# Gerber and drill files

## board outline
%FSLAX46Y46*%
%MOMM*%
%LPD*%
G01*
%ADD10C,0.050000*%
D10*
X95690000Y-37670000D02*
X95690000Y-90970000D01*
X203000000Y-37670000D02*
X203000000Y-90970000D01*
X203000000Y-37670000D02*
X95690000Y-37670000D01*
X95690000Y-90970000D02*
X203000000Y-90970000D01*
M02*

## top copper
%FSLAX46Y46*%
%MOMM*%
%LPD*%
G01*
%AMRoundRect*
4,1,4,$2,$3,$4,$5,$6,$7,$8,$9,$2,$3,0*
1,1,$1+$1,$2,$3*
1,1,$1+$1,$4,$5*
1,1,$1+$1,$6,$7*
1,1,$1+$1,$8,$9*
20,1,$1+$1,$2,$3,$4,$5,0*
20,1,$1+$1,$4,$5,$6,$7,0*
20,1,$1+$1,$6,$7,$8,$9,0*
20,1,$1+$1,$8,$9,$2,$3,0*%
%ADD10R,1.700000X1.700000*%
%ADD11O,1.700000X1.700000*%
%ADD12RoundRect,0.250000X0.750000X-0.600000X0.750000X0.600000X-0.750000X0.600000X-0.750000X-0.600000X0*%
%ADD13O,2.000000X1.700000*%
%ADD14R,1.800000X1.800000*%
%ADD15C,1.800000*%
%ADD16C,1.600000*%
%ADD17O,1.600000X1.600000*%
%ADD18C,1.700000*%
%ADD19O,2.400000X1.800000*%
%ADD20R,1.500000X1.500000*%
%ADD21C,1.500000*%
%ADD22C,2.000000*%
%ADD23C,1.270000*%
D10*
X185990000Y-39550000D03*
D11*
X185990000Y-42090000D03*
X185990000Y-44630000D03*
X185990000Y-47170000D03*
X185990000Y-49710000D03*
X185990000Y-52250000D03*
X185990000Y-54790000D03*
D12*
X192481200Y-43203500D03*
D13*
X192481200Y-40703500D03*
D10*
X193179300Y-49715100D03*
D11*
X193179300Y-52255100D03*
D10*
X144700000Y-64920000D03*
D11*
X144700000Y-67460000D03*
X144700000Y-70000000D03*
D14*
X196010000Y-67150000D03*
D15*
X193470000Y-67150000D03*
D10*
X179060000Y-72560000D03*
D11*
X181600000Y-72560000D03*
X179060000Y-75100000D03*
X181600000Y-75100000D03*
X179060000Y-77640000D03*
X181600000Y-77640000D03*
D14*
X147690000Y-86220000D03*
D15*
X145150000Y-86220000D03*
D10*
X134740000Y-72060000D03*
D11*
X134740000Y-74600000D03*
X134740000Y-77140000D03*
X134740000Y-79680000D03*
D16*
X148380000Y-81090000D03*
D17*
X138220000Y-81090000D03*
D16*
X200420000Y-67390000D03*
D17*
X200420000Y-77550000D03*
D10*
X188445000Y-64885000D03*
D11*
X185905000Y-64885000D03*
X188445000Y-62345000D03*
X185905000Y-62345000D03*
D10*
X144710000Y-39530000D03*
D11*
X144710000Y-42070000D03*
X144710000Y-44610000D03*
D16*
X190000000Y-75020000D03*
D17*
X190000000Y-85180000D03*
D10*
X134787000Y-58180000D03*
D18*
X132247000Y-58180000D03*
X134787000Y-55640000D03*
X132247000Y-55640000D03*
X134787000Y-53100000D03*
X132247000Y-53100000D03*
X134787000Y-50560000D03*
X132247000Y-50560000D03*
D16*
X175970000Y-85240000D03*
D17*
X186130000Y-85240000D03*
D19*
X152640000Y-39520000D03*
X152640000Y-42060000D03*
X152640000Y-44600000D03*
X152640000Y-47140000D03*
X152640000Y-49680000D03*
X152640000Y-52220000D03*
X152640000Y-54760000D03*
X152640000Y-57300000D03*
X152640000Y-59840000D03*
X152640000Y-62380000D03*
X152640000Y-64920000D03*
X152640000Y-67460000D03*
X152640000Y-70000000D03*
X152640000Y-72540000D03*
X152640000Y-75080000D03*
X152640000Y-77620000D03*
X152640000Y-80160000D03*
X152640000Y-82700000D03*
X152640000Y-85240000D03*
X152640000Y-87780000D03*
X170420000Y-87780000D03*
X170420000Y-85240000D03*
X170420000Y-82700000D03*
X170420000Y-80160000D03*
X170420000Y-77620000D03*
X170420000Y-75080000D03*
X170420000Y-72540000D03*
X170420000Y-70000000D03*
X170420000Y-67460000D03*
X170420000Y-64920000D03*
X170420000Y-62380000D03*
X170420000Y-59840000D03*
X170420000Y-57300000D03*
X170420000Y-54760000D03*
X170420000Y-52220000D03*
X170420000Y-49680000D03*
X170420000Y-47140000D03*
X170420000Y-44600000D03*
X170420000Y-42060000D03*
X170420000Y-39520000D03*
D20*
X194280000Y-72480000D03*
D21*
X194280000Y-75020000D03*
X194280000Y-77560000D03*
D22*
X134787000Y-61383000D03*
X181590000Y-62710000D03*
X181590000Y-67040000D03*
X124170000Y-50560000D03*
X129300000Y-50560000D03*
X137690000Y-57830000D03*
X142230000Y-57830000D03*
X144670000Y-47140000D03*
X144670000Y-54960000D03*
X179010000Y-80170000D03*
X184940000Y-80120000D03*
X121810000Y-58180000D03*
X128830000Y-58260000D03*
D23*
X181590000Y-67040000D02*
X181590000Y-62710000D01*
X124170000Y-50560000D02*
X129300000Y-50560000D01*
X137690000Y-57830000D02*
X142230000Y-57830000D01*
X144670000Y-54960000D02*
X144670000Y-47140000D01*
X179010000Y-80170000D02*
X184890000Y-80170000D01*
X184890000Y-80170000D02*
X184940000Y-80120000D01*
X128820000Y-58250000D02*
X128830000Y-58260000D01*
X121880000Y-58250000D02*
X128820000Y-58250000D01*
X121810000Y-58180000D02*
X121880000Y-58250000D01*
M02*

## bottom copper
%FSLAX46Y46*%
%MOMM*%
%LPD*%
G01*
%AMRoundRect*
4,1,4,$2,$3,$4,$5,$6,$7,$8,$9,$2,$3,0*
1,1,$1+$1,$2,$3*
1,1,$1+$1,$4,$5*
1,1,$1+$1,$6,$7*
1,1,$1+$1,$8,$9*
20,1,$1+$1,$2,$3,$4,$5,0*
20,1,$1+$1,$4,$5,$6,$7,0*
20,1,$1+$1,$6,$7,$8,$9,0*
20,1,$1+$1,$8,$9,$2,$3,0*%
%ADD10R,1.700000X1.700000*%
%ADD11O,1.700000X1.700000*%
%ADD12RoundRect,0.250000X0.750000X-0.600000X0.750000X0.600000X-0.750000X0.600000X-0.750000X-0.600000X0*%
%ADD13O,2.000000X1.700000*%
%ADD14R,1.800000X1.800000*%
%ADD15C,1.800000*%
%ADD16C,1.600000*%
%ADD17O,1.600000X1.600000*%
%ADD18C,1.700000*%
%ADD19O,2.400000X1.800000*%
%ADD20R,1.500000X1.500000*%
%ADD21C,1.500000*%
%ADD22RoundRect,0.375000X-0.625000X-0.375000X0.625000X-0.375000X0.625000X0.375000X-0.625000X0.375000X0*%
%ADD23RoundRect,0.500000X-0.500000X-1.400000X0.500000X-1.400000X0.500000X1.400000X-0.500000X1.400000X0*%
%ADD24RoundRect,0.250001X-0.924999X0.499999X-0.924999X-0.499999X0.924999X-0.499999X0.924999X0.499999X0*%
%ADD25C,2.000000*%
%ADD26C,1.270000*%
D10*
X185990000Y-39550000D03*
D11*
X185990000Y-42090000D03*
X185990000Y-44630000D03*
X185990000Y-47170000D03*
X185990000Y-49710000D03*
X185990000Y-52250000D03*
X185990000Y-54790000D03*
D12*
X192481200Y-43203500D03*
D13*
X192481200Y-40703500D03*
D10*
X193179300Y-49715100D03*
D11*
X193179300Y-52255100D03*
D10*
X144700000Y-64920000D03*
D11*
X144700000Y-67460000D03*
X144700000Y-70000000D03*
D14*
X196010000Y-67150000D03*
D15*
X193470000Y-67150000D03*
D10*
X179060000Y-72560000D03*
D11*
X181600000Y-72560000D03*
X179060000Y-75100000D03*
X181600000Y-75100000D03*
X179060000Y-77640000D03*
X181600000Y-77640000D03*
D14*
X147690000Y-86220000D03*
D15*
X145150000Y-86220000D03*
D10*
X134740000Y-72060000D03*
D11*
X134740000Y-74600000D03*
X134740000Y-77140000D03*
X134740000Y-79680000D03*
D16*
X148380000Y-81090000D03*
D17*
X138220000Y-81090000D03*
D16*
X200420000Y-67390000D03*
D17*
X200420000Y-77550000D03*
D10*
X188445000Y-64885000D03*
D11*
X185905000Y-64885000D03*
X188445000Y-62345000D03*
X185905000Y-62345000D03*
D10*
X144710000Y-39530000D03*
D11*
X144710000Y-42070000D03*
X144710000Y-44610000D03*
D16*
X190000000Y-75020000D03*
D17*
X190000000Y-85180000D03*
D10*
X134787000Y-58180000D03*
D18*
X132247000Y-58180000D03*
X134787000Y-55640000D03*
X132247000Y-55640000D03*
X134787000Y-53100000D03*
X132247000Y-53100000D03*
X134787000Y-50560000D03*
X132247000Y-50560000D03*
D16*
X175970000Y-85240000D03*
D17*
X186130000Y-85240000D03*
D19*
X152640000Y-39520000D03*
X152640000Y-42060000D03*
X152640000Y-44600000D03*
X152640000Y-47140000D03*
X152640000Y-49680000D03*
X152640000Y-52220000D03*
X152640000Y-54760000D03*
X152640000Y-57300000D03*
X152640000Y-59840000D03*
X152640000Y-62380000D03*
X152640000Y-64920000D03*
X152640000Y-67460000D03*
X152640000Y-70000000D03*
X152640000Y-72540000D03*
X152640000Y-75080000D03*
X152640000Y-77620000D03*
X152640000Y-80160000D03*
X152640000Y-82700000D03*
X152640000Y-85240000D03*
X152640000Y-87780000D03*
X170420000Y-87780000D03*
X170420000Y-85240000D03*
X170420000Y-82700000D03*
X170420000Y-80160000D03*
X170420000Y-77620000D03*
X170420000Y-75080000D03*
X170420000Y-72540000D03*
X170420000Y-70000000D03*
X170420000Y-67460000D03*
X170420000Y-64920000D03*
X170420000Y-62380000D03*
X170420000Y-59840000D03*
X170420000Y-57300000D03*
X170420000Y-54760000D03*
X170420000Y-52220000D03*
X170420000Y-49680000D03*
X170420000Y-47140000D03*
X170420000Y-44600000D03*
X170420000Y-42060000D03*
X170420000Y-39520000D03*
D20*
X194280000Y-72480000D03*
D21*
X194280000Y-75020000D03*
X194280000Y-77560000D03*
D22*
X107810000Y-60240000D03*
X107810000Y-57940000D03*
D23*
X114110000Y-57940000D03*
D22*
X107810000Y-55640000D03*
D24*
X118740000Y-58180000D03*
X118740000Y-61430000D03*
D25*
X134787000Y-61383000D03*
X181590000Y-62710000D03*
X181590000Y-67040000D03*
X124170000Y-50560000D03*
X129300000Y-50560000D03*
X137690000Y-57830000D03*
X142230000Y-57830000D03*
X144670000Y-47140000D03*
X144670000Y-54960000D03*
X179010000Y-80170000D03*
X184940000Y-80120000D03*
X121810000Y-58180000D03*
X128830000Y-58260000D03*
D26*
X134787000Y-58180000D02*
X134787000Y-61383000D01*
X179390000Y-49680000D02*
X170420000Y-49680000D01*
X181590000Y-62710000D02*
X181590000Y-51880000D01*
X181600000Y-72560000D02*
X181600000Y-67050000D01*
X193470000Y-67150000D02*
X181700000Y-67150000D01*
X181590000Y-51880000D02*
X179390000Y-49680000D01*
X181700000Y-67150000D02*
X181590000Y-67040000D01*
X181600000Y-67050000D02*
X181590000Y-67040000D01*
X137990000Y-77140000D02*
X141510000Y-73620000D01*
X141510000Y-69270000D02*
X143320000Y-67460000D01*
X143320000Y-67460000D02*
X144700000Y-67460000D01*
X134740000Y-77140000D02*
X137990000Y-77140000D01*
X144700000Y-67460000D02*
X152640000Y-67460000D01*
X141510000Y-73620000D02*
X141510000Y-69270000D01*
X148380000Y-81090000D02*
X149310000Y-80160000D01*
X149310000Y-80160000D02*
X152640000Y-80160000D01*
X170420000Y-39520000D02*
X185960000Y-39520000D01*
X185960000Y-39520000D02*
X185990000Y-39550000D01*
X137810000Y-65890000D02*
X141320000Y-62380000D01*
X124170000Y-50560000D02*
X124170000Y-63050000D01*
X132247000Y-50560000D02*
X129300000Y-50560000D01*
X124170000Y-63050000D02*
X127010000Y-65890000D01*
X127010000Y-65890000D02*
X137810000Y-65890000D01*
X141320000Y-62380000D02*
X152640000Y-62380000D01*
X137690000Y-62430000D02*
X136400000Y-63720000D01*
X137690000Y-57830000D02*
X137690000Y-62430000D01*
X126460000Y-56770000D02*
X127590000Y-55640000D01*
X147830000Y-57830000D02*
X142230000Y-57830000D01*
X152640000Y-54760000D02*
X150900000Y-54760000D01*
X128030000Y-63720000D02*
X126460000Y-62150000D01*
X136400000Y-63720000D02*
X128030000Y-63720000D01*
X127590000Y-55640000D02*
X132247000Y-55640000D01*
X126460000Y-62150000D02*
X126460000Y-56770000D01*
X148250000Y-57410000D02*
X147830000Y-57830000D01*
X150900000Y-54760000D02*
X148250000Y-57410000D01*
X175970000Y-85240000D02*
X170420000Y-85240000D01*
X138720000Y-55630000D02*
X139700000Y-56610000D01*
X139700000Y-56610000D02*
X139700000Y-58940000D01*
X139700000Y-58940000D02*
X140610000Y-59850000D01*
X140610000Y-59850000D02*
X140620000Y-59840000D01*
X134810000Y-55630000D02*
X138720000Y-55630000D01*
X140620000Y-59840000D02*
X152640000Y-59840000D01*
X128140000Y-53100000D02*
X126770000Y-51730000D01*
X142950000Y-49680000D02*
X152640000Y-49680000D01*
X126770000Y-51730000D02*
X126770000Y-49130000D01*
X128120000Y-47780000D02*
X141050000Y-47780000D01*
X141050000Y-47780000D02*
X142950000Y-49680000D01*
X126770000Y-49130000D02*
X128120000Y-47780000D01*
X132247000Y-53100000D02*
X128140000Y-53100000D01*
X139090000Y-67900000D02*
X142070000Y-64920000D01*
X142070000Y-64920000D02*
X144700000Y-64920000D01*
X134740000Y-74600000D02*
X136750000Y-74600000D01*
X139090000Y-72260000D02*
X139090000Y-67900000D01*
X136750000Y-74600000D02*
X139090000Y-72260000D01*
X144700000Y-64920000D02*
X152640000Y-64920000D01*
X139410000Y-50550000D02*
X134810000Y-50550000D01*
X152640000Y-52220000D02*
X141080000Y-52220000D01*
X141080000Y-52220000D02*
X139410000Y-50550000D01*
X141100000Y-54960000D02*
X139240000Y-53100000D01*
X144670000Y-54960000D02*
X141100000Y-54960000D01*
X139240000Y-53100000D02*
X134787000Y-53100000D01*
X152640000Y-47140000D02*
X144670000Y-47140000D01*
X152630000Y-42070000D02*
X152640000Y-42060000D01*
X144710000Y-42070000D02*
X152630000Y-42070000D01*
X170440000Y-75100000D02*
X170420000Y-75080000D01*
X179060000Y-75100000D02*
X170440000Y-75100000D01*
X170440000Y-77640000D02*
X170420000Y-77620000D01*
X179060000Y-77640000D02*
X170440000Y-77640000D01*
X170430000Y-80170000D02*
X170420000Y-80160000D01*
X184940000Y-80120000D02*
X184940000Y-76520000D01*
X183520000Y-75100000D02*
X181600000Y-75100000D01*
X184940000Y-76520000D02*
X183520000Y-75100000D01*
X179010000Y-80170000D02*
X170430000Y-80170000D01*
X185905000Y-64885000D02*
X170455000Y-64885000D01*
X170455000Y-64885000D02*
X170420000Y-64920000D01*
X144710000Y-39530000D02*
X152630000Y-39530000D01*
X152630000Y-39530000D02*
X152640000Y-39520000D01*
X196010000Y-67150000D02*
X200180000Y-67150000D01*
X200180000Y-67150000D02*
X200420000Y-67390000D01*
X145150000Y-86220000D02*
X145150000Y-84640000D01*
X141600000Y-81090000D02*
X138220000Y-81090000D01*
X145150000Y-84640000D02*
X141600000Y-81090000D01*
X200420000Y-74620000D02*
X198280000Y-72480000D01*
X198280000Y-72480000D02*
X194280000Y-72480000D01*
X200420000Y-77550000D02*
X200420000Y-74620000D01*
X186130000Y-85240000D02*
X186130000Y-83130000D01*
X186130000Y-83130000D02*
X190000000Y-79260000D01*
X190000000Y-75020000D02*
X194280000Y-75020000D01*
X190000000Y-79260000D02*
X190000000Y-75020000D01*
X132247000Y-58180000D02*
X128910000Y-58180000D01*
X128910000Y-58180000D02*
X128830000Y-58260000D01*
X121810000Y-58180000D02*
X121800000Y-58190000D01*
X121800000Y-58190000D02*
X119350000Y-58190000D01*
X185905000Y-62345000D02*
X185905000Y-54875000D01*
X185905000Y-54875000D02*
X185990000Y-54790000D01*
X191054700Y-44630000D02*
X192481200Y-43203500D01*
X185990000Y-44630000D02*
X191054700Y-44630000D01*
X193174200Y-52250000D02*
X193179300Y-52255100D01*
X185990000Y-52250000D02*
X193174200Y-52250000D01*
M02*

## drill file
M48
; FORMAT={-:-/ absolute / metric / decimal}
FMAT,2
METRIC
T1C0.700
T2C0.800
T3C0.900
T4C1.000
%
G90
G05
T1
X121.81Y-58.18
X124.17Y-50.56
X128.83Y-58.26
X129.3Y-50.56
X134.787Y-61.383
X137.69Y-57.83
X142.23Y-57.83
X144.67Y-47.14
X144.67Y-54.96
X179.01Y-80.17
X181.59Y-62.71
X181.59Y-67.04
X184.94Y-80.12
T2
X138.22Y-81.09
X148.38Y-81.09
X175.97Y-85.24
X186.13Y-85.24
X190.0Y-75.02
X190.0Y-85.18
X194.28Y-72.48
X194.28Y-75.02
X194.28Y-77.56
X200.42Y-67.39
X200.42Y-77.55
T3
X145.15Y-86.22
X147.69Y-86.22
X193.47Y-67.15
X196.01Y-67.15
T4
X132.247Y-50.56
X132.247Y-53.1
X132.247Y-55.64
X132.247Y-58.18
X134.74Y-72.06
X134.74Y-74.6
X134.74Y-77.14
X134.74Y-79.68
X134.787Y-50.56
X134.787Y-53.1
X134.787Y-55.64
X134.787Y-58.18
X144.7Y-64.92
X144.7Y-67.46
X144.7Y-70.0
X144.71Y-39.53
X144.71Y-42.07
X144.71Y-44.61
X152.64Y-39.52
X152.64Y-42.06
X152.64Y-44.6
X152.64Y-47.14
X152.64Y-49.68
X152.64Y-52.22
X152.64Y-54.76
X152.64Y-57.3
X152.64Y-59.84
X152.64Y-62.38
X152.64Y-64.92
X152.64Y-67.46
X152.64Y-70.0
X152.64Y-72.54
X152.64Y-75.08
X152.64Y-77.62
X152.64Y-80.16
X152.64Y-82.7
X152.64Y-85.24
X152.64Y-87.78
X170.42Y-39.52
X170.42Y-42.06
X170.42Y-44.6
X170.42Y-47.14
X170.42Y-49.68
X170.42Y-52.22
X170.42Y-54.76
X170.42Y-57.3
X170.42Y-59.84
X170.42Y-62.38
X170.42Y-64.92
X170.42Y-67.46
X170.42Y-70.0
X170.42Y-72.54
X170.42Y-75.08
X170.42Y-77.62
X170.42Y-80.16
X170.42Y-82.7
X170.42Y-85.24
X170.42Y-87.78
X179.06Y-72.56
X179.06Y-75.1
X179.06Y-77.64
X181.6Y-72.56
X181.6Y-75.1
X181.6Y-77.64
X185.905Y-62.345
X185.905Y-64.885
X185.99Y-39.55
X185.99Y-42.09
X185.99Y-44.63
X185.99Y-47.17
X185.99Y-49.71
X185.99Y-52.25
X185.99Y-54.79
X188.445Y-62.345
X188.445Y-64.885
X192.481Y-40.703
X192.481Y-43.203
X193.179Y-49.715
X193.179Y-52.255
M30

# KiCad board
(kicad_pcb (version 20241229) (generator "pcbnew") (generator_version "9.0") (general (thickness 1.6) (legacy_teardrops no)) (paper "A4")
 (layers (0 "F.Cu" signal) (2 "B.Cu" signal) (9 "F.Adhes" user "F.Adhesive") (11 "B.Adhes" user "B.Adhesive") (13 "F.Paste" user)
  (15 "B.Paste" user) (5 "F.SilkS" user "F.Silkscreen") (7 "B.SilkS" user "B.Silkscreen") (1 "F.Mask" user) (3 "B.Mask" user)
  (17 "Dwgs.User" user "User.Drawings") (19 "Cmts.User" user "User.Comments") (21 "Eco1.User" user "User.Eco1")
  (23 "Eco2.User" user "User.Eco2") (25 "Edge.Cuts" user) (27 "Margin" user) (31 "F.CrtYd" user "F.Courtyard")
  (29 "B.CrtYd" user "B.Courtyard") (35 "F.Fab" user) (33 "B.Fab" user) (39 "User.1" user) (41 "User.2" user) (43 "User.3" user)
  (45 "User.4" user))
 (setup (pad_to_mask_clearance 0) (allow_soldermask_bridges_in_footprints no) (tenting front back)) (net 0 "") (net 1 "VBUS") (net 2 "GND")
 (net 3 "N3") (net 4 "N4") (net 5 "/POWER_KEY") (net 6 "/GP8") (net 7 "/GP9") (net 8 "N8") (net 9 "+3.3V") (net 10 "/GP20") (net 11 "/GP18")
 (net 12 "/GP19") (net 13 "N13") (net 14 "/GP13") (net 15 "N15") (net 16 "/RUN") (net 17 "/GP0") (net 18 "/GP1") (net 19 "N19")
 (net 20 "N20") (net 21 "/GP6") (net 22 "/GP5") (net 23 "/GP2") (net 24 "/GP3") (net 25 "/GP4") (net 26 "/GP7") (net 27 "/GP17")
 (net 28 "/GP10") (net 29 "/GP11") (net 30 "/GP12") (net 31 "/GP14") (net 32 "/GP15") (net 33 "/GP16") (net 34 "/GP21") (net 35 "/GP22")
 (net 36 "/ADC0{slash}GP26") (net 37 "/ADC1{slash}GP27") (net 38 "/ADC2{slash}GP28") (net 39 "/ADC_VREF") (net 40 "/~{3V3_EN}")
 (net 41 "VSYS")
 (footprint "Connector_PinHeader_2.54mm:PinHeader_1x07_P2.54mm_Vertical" (layer "F.Cu") (at 185.99 39.55)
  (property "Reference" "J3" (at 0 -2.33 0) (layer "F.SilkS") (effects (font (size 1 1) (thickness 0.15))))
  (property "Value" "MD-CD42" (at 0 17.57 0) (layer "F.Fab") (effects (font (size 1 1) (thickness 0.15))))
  (pad "1" thru_hole rect (at 0 0) (size 1.7 1.7) (drill 1) (layers "*.Cu" "*.Mask") (remove_unused_layers no) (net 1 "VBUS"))
  (pad "2" thru_hole oval (at 0 2.54) (size 1.7 1.7) (drill 1) (layers "*.Cu" "*.Mask") (remove_unused_layers no) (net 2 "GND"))
  (pad "3" thru_hole oval (at 0 5.08) (size 1.7 1.7) (drill 1) (layers "*.Cu" "*.Mask") (remove_unused_layers no) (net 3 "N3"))
  (pad "4" thru_hole oval (at 0 7.62) (size 1.7 1.7) (drill 1) (layers "*.Cu" "*.Mask") (remove_unused_layers no) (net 2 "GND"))
  (pad "5" thru_hole oval (at 0 10.16) (size 1.7 1.7) (drill 1) (layers "*.Cu" "*.Mask") (remove_unused_layers no) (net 2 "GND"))
  (pad "6" thru_hole oval (at 0 12.7) (size 1.7 1.7) (drill 1) (layers "*.Cu" "*.Mask") (remove_unused_layers no) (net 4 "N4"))
  (pad "7" thru_hole oval (at 0 15.24) (size 1.7 1.7) (drill 1) (layers "*.Cu" "*.Mask") (remove_unused_layers no) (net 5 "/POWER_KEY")))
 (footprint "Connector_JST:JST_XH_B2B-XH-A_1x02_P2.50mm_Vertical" (layer "F.Cu") (at 192.4812 43.2035 90)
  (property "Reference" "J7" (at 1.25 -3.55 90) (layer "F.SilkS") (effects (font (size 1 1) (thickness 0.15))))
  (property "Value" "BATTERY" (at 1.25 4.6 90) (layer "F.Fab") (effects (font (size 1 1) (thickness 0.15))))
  (pad "1" thru_hole roundrect (at 0 0 90) (size 1.7 2) (drill 1) (layers "*.Cu" "*.Mask") (remove_unused_layers no)
   (roundrect_rratio 0.147059) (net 3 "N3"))
  (pad "2" thru_hole oval (at 2.5 0 90) (size 1.7 2) (drill 1) (layers "*.Cu" "*.Mask") (remove_unused_layers no) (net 2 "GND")))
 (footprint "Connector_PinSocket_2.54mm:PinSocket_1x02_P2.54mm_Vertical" (layer "F.Cu") (at 193.1793 49.7151)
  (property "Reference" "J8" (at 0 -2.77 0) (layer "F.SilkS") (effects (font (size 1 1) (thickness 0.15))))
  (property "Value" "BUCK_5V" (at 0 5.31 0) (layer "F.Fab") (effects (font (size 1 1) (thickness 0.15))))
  (pad "1" thru_hole rect (at 0 0) (size 1.7 1.7) (drill 1) (layers "*.Cu" "*.Mask") (remove_unused_layers no) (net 2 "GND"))
  (pad "2" thru_hole oval (at 0 2.54) (size 1.7 1.7) (drill 1) (layers "*.Cu" "*.Mask") (remove_unused_layers no) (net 4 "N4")))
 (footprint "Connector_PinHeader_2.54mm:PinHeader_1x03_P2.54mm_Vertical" (layer "F.Cu") (at 144.7 64.92)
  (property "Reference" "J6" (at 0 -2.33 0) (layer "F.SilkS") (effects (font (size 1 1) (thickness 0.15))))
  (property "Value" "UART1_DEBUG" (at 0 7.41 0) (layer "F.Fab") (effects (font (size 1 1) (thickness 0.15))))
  (pad "1" thru_hole rect (at 0 0) (size 1.7 1.7) (drill 1) (layers "*.Cu" "*.Mask") (remove_unused_layers no) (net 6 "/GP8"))
  (pad "2" thru_hole oval (at 0 2.54) (size 1.7 1.7) (drill 1) (layers "*.Cu" "*.Mask") (remove_unused_layers no) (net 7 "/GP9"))
  (pad "3" thru_hole oval (at 0 5.08) (size 1.7 1.7) (drill 1) (layers "*.Cu" "*.Mask") (remove_unused_layers no) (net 2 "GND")))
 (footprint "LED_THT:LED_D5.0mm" (layer "F.Cu") (at 196.01 67.15 180)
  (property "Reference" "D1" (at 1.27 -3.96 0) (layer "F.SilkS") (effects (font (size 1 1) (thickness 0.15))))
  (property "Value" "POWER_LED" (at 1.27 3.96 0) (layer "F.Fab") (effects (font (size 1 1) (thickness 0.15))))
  (pad "1" thru_hole rect (at 0 0 180) (size 1.8 1.8) (drill 0.9) (layers "*.Cu" "*.Mask") (remove_unused_layers no) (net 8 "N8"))
  (pad "2" thru_hole circle (at 2.54 0 180) (size 1.8 1.8) (drill 0.9) (layers "*.Cu" "*.Mask") (remove_unused_layers no) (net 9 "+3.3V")))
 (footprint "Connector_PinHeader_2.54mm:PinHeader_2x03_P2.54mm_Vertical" (layer "F.Cu") (at 179.06 72.56)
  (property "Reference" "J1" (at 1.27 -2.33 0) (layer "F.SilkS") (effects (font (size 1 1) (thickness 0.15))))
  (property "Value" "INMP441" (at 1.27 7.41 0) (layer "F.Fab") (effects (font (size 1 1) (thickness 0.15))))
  (pad "1" thru_hole rect (at 0 0) (size 1.7 1.7) (drill 1) (layers "*.Cu" "*.Mask") (remove_unused_layers no) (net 2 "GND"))
  (pad "2" thru_hole oval (at 2.54 0) (size 1.7 1.7) (drill 1) (layers "*.Cu" "*.Mask") (remove_unused_layers no) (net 9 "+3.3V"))
  (pad "3" thru_hole oval (at 0 2.54) (size 1.7 1.7) (drill 1) (layers "*.Cu" "*.Mask") (remove_unused_layers no) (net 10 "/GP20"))
  (pad "4" thru_hole oval (at 2.54 2.54) (size 1.7 1.7) (drill 1) (layers "*.Cu" "*.Mask") (remove_unused_layers no) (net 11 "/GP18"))
  (pad "5" thru_hole oval (at 0 5.08) (size 1.7 1.7) (drill 1) (layers "*.Cu" "*.Mask") (remove_unused_layers no) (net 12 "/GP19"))
  (pad "6" thru_hole oval (at 2.54 5.08) (size 1.7 1.7) (drill 1) (layers "*.Cu" "*.Mask") (remove_unused_layers no) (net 2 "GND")))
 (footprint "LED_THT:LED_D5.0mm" (layer "F.Cu") (at 147.69 86.22 180)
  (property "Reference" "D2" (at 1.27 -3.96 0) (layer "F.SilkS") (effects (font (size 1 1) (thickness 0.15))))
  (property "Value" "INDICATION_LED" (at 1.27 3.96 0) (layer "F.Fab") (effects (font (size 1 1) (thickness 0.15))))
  (pad "1" thru_hole rect (at 0 0 180) (size 1.8 1.8) (drill 0.9) (layers "*.Cu" "*.Mask") (remove_unused_layers no) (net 2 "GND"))
  (pad "2" thru_hole circle (at 2.54 0 180) (size 1.8 1.8) (drill 0.9) (layers "*.Cu" "*.Mask") (remove_unused_layers no) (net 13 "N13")))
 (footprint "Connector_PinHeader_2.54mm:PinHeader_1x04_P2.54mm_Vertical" (layer "F.Cu") (at 134.74 72.06)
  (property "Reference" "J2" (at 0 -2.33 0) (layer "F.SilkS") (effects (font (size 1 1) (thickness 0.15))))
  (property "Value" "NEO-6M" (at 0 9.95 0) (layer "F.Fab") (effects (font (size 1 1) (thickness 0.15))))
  (pad "1" thru_hole rect (at 0 0) (size 1.7 1.7) (drill 1) (layers "*.Cu" "*.Mask") (remove_unused_layers no) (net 9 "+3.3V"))
  (pad "2" thru_hole oval (at 0 2.54) (size 1.7 1.7) (drill 1) (layers "*.Cu" "*.Mask") (remove_unused_layers no) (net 6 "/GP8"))
  (pad "3" thru_hole oval (at 0 5.08) (size 1.7 1.7) (drill 1) (layers "*.Cu" "*.Mask") (remove_unused_layers no) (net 7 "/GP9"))
  (pad "4" thru_hole oval (at 0 7.62) (size 1.7 1.7) (drill 1) (layers "*.Cu" "*.Mask") (remove_unused_layers no) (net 2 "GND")))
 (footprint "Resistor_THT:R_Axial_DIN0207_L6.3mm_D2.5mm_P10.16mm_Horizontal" (layer "F.Cu") (at 148.38 81.09 180)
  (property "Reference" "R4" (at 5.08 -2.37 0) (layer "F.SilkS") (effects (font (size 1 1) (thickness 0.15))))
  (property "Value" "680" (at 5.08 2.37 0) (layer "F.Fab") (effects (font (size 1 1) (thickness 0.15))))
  (pad "1" thru_hole circle (at 0 0 180) (size 1.6 1.6) (drill 0.8) (layers "*.Cu" "*.Mask") (remove_unused_layers no) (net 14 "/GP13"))
  (pad "2" thru_hole oval (at 10.16 0 180) (size 1.6 1.6) (drill 0.8) (layers "*.Cu" "*.Mask") (remove_unused_layers no) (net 13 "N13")))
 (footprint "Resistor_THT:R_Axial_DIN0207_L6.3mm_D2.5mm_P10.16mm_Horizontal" (layer "F.Cu") (at 200.42 67.39 -90)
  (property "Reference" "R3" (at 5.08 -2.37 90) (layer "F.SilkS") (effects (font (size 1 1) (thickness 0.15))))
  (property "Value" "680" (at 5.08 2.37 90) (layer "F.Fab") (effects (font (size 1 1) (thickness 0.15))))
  (pad "1" thru_hole circle (at 0 0 270) (size 1.6 1.6) (drill 0.8) (layers "*.Cu" "*.Mask") (remove_unused_layers no) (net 8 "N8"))
  (pad "2" thru_hole oval (at 10.16 0 270) (size 1.6 1.6) (drill 0.8) (layers "*.Cu" "*.Mask") (remove_unused_layers no) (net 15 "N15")))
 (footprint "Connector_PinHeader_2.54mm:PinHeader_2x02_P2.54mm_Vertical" (layer "F.Cu") (at 188.445 64.885 180)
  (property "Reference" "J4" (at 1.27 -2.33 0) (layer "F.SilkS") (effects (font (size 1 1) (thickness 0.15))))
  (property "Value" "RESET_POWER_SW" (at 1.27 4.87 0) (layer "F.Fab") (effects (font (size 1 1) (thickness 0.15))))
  (pad "1" thru_hole rect (at 0 0 180) (size 1.7 1.7) (drill 1) (layers "*.Cu" "*.Mask") (remove_unused_layers no) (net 2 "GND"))
  (pad "2" thru_hole oval (at 2.54 0 180) (size 1.7 1.7) (drill 1) (layers "*.Cu" "*.Mask") (remove_unused_layers no) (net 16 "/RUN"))
  (pad "3" thru_hole oval (at 0 2.54 180) (size 1.7 1.7) (drill 1) (layers "*.Cu" "*.Mask") (remove_unused_layers no) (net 2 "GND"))
  (pad "4" thru_hole oval (at 2.54 2.54 180) (size 1.7 1.7) (drill 1) (layers "*.Cu" "*.Mask") (remove_unused_layers no)
   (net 5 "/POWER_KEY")))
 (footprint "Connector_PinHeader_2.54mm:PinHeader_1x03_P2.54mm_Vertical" (layer "F.Cu") (at 144.71 39.53)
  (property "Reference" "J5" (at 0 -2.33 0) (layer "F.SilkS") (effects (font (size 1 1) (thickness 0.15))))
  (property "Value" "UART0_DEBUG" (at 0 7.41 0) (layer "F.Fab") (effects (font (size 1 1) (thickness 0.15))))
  (pad "1" thru_hole rect (at 0 0) (size 1.7 1.7) (drill 1) (layers "*.Cu" "*.Mask") (remove_unused_layers no) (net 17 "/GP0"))
  (pad "2" thru_hole oval (at 0 2.54) (size 1.7 1.7) (drill 1) (layers "*.Cu" "*.Mask") (remove_unused_layers no) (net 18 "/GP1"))
  (pad "3" thru_hole oval (at 0 5.08) (size 1.7 1.7) (drill 1) (layers "*.Cu" "*.Mask") (remove_unused_layers no) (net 2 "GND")))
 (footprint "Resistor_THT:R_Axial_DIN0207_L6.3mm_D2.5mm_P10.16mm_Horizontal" (layer "F.Cu") (at 190 75.02 -90)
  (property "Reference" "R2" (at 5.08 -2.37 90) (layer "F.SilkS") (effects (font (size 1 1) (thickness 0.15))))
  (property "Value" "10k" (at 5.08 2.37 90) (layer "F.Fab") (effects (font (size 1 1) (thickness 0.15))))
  (pad "1" thru_hole circle (at 0 0 270) (size 1.6 1.6) (drill 0.8) (layers "*.Cu" "*.Mask") (remove_unused_layers no) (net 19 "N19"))
  (pad "2" thru_hole oval (at 10.16 0 270) (size 1.6 1.6) (drill 0.8) (layers "*.Cu" "*.Mask") (remove_unused_layers no) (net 2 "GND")))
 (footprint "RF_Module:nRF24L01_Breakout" (layer "F.Cu") (at 136.287 54.39 180)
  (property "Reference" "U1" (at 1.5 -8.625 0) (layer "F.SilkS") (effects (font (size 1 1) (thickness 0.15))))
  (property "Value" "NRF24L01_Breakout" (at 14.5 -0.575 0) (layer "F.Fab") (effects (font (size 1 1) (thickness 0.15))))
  (pad "1" thru_hole rect (at 1.5 -3.79 180) (size 1.7 1.7) (drill 1) (layers "*.Cu" "*.Mask") (remove_unused_layers no) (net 2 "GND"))
  (pad "2" thru_hole circle (at 4.04 -3.79 180) (size 1.7 1.7) (drill 1) (layers "*.Cu" "*.Mask") (remove_unused_layers no) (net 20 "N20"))
  (pad "3" thru_hole circle (at 1.5 -1.25 180) (size 1.7 1.7) (drill 1) (layers "*.Cu" "*.Mask") (remove_unused_layers no) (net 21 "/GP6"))
  (pad "4" thru_hole circle (at 4.04 -1.25 180) (size 1.7 1.7) (drill 1) (layers "*.Cu" "*.Mask") (remove_unused_layers no) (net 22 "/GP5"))
  (pad "5" thru_hole circle (at 1.5 1.29 180) (size 1.7 1.7) (drill 1) (layers "*.Cu" "*.Mask") (remove_unused_layers no) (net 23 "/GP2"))
  (pad "6" thru_hole circle (at 4.04 1.29 180) (size 1.7 1.7) (drill 1) (layers "*.Cu" "*.Mask") (remove_unused_layers no) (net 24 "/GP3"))
  (pad "7" thru_hole circle (at 1.5 3.83 180) (size 1.7 1.7) (drill 1) (layers "*.Cu" "*.Mask") (remove_unused_layers no) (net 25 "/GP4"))
  (pad "8" thru_hole circle (at 4.04 3.83 180) (size 1.7 1.7) (drill 1) (layers "*.Cu" "*.Mask") (remove_unused_layers no) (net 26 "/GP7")))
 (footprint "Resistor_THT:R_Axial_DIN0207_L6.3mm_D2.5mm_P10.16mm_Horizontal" (layer "F.Cu") (at 175.97 85.24)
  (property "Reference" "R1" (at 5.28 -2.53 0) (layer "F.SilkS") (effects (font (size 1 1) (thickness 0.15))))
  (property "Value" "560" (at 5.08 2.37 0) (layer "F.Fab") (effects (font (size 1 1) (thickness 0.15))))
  (pad "1" thru_hole circle (at 0 0) (size 1.6 1.6) (drill 0.8) (layers "*.Cu" "*.Mask") (remove_unused_layers no) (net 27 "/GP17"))
  (pad "2" thru_hole oval (at 10.16 0) (size 1.6 1.6) (drill 0.8) (layers "*.Cu" "*.Mask") (remove_unused_layers no) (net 19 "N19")))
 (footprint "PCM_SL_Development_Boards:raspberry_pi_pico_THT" (layer "F.Cu") (at 152.64 39.52)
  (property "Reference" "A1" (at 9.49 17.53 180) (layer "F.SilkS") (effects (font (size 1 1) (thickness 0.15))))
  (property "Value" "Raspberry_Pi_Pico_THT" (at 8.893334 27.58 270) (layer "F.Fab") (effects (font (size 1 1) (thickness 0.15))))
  (pad "1" thru_hole oval (at 0 0 270) (size 1.8 2.4) (drill 1) (layers "*.Cu" "*.Mask") (remove_unused_layers no) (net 17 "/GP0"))
  (pad "2" thru_hole oval (at 0 2.54 270) (size 1.8 2.4) (drill 1) (layers "*.Cu" "*.Mask") (remove_unused_layers no) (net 18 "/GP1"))
  (pad "3" thru_hole oval (at 0 5.08 270) (size 1.8 2.4) (drill 1) (layers "*.Cu" "*.Mask") (remove_unused_layers no) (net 2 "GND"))
  (pad "4" thru_hole oval (at 0 7.62 270) (size 1.8 2.4) (drill 1) (layers "*.Cu" "*.Mask") (remove_unused_layers no) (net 23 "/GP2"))
  (pad "5" thru_hole oval (at 0 10.16 270) (size 1.8 2.4) (drill 1) (layers "*.Cu" "*.Mask") (remove_unused_layers no) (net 24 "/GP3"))
  (pad "6" thru_hole oval (at 0 12.7 270) (size 1.8 2.4) (drill 1) (layers "*.Cu" "*.Mask") (remove_unused_layers no) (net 25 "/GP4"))
  (pad "7" thru_hole oval (at 0 15.24 270) (size 1.8 2.4) (drill 1) (layers "*.Cu" "*.Mask") (remove_unused_layers no) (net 22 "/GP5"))
  (pad "8" thru_hole oval (at 0 17.78 270) (size 1.8 2.4) (drill 1) (layers "*.Cu" "*.Mask") (remove_unused_layers no) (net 2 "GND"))
  (pad "9" thru_hole oval (at 0 20.32 270) (size 1.8 2.4) (drill 1) (layers "*.Cu" "*.Mask") (remove_unused_layers no) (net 21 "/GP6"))
  (pad "10" thru_hole oval (at 0 22.86 270) (size 1.8 2.4) (drill 1) (layers "*.Cu" "*.Mask") (remove_unused_layers no) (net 26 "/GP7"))
  (pad "11" thru_hole oval (at 0 25.4 270) (size 1.8 2.4) (drill 1) (layers "*.Cu" "*.Mask") (remove_unused_layers no) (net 6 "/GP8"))
  (pad "12" thru_hole oval (at 0 27.94 270) (size 1.8 2.4) (drill 1) (layers "*.Cu" "*.Mask") (remove_unused_layers no) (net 7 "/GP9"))
  (pad "13" thru_hole oval (at 0 30.48 270) (size 1.8 2.4) (drill 1) (layers "*.Cu" "*.Mask") (remove_unused_layers no) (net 2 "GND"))
  (pad "14" thru_hole oval (at 0 33.02 270) (size 1.8 2.4) (drill 1) (layers "*.Cu" "*.Mask") (remove_unused_layers no) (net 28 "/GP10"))
  (pad "15" thru_hole oval (at 0 35.56 270) (size 1.8 2.4) (drill 1) (layers "*.Cu" "*.Mask") (remove_unused_layers no) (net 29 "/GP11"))
  (pad "16" thru_hole oval (at 0 38.1 270) (size 1.8 2.4) (drill 1) (layers "*.Cu" "*.Mask") (remove_unused_layers no) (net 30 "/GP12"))
  (pad "17" thru_hole oval (at 0 40.64 270) (size 1.8 2.4) (drill 1) (layers "*.Cu" "*.Mask") (remove_unused_layers no) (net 14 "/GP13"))
  (pad "18" thru_hole oval (at 0 43.18 270) (size 1.8 2.4) (drill 1) (layers "*.Cu" "*.Mask") (remove_unused_layers no) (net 2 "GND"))
  (pad "19" thru_hole oval (at 0 45.72 270) (size 1.8 2.4) (drill 1) (layers "*.Cu" "*.Mask") (remove_unused_layers no) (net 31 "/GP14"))
  (pad "20" thru_hole oval (at 0 48.26 270) (size 1.8 2.4) (drill 1) (layers "*.Cu" "*.Mask") (remove_unused_layers no) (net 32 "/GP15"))
  (pad "21" thru_hole oval (at 17.78 48.26 270) (size 1.8 2.4) (drill 1) (layers "*.Cu" "*.Mask") (remove_unused_layers no) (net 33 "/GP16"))
  (pad "22" thru_hole oval (at 17.78 45.72 270) (size 1.8 2.4) (drill 1) (layers "*.Cu" "*.Mask") (remove_unused_layers no) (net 27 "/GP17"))
  (pad "23" thru_hole oval (at 17.78 43.18 270) (size 1.8 2.4) (drill 1) (layers "*.Cu" "*.Mask") (remove_unused_layers no) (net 2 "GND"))
  (pad "24" thru_hole oval (at 17.78 40.64 270) (size 1.8 2.4) (drill 1) (layers "*.Cu" "*.Mask") (remove_unused_layers no) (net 11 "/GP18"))
  (pad "25" thru_hole oval (at 17.78 38.1 270) (size 1.8 2.4) (drill 1) (layers "*.Cu" "*.Mask") (remove_unused_layers no) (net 12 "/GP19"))
  (pad "26" thru_hole oval (at 17.78 35.56 270) (size 1.8 2.4) (drill 1) (layers "*.Cu" "*.Mask") (remove_unused_layers no) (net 10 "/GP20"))
  (pad "27" thru_hole oval (at 17.78 33.02 270) (size 1.8 2.4) (drill 1) (layers "*.Cu" "*.Mask") (remove_unused_layers no) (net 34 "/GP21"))
  (pad "28" thru_hole oval (at 17.78 30.48 270) (size 1.8 2.4) (drill 1) (layers "*.Cu" "*.Mask") (remove_unused_layers no) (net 2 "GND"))
  (pad "29" thru_hole oval (at 17.78 27.94 270) (size 1.8 2.4) (drill 1) (layers "*.Cu" "*.Mask") (remove_unused_layers no) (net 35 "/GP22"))
  (pad "30" thru_hole oval (at 17.78 25.4 270) (size 1.8 2.4) (drill 1) (layers "*.Cu" "*.Mask") (remove_unused_layers no) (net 16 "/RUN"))
  (pad "31" thru_hole oval (at 17.78 22.86 270) (size 1.8 2.4) (drill 1) (layers "*.Cu" "*.Mask") (remove_unused_layers no)
   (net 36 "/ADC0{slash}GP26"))
  (pad "32" thru_hole oval (at 17.78 20.32 270) (size 1.8 2.4) (drill 1) (layers "*.Cu" "*.Mask") (remove_unused_layers no)
   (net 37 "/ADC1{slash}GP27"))
  (pad "33" thru_hole oval (at 17.78 17.78 270) (size 1.8 2.4) (drill 1) (layers "*.Cu" "*.Mask") (remove_unused_layers no) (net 2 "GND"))
  (pad "34" thru_hole oval (at 17.78 15.24 270) (size 1.8 2.4) (drill 1) (layers "*.Cu" "*.Mask") (remove_unused_layers no)
   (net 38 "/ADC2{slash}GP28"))
  (pad "35" thru_hole oval (at 17.78 12.7 270) (size 1.8 2.4) (drill 1) (layers "*.Cu" "*.Mask") (remove_unused_layers no)
   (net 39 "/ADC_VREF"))
  (pad "36" thru_hole oval (at 17.78 10.16 270) (size 1.8 2.4) (drill 1) (layers "*.Cu" "*.Mask") (remove_unused_layers no) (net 9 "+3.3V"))
  (pad "37" thru_hole oval (at 17.78 7.62 270) (size 1.8 2.4) (drill 1) (layers "*.Cu" "*.Mask") (remove_unused_layers no)
   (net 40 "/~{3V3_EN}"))
  (pad "38" thru_hole oval (at 17.78 5.08 270) (size 1.8 2.4) (drill 1) (layers "*.Cu" "*.Mask") (remove_unused_layers no) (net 2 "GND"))
  (pad "39" thru_hole oval (at 17.78 2.54 270) (size 1.8 2.4) (drill 1) (layers "*.Cu" "*.Mask") (remove_unused_layers no) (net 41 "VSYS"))
  (pad "40" thru_hole oval (at 17.78 0 270) (size 1.8 2.4) (drill 1) (layers "*.Cu" "*.Mask") (remove_unused_layers no) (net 1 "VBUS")))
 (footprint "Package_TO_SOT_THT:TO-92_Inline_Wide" (layer "F.Cu") (at 194.28 72.48 -90)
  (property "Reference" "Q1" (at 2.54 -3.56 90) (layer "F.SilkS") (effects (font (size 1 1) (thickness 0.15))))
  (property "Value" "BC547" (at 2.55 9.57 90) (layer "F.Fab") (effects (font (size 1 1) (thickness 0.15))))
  (pad "1" thru_hole rect (at 0 0 270) (size 1.5 1.5) (drill 0.8) (layers "*.Cu" "*.Mask") (remove_unused_layers no) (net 15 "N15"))
  (pad "2" thru_hole circle (at 2.54 0 270) (size 1.5 1.5) (drill 0.8) (layers "*.Cu" "*.Mask") (remove_unused_layers no) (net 19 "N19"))
  (pad "3" thru_hole circle (at 5.08 0 270) (size 1.5 1.5) (drill 0.8) (layers "*.Cu" "*.Mask") (remove_unused_layers no) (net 2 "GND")))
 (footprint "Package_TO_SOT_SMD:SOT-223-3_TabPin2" (layer "B.Cu") (at 110.96 57.94)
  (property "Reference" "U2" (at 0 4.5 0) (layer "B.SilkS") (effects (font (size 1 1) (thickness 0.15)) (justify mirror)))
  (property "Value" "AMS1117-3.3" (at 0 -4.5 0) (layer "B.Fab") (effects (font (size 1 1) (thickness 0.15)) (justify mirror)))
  (pad "1" smd roundrect (at -3.15 2.3) (size 2 1.5) (layers "B.Cu" "B.Mask" "B.Paste") (roundrect_rratio 0.25) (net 2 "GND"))
  (pad "2" smd roundrect (at -3.15 0) (size 2 1.5) (layers "B.Cu" "B.Mask" "B.Paste") (roundrect_rratio 0.25) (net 20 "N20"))
  (pad "2" smd roundrect (at 3.15 0) (size 2 3.8) (layers "B.Cu" "B.Mask" "B.Paste") (roundrect_rratio 0.25) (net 20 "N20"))
  (pad "3" smd roundrect (at -3.15 -2.3) (size 2 1.5) (layers "B.Cu" "B.Mask" "B.Paste") (roundrect_rratio 0.25) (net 1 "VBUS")))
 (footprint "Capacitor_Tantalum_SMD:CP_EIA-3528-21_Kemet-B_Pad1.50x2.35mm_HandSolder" (layer "B.Cu") (at 118.74 59.805 -90)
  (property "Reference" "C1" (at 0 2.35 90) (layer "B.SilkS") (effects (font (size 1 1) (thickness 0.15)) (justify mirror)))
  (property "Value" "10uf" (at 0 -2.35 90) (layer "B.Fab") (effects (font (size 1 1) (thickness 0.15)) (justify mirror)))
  (pad "1" smd roundrect (at -1.625 0 270) (size 1.5 2.35) (layers "B.Cu" "B.Mask" "B.Paste") (roundrect_rratio 0.166667) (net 20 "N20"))
  (pad "2" smd roundrect (at 1.625 0 270) (size 1.5 2.35) (layers "B.Cu" "B.Mask" "B.Paste") (roundrect_rratio 0.166667) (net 2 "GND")))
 (gr_line (start 95.69 37.67) (end 95.69 90.97) (stroke (width 0.05) (type default)) (layer "Edge.Cuts"))
 (gr_line (start 203 37.67) (end 203 90.97) (stroke (width 0.05) (type default)) (layer "Edge.Cuts"))
 (gr_line (start 203 37.67) (end 95.69 37.67) (stroke (width 0.05) (type default)) (layer "Edge.Cuts"))
 (gr_line (start 95.69 90.97) (end 203 90.97) (stroke (width 0.05) (type default)) (layer "Edge.Cuts"))
 (via (at 134.787 61.383) (size 2) (drill 0.7) (layers "F.Cu" "B.Cu") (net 2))
 (segment (start 134.787 58.18) (end 134.787 61.383) (width 1.27) (layer "B.Cu") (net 2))
 (segment (start 181.59 67.04) (end 181.59 62.71) (width 1.27) (layer "F.Cu") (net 9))
 (via (at 181.59 62.71) (size 2) (drill 0.7) (layers "F.Cu" "B.Cu") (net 9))
 (via (at 181.59 67.04) (size 2) (drill 0.7) (layers "F.Cu" "B.Cu") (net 9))
 (segment (start 179.39 49.68) (end 170.42 49.68) (width 1.27) (layer "B.Cu") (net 9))
 (segment (start 181.59 62.71) (end 181.59 51.88) (width 1.27) (layer "B.Cu") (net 9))
 (segment (start 181.6 72.56) (end 181.6 67.05) (width 1.27) (layer "B.Cu") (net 9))
 (segment (start 193.47 67.15) (end 181.7 67.15) (width 1.27) (layer "B.Cu") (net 9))
 (segment (start 181.59 51.88) (end 179.39 49.68) (width 1.27) (layer "B.Cu") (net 9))
 (segment (start 181.7 67.15) (end 181.59 67.04) (width 1.27) (layer "B.Cu") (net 9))
 (segment (start 181.6 67.05) (end 181.59 67.04) (width 1.27) (layer "B.Cu") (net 9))
 (segment (start 137.99 77.14) (end 141.51 73.62) (width 1.27) (layer "B.Cu") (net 7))
 (segment (start 141.51 69.27) (end 143.32 67.46) (width 1.27) (layer "B.Cu") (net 7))
 (segment (start 143.32 67.46) (end 144.7 67.46) (width 1.27) (layer "B.Cu") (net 7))
 (segment (start 134.74 77.14) (end 137.99 77.14) (width 1.27) (layer "B.Cu") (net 7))
 (segment (start 144.7 67.46) (end 152.64 67.46) (width 1.27) (layer "B.Cu") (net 7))
 (segment (start 141.51 73.62) (end 141.51 69.27) (width 1.27) (layer "B.Cu") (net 7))
 (segment (start 148.38 81.09) (end 149.31 80.16) (width 1.27) (layer "B.Cu") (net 14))
 (segment (start 149.31 80.16) (end 152.64 80.16) (width 1.27) (layer "B.Cu") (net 14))
 (segment (start 170.42 39.52) (end 185.96 39.52) (width 1.27) (layer "B.Cu") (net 1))
 (segment (start 185.96 39.52) (end 185.99 39.55) (width 1.27) (layer "B.Cu") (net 1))
 (segment (start 124.17 50.56) (end 129.3 50.56) (width 1.27) (layer "F.Cu") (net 26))
 (via (at 124.17 50.56) (size 2) (drill 0.7) (layers "F.Cu" "B.Cu") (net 26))
 (via (at 129.3 50.56) (size 2) (drill 0.7) (layers "F.Cu" "B.Cu") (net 26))
 (segment (start 137.81 65.89) (end 141.32 62.38) (width 1.27) (layer "B.Cu") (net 26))
 (segment (start 124.17 50.56) (end 124.17 63.05) (width 1.27) (layer "B.Cu") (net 26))
 (segment (start 132.247 50.56) (end 129.3 50.56) (width 1.27) (layer "B.Cu") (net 26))
 (segment (start 124.17 63.05) (end 127.01 65.89) (width 1.27) (layer "B.Cu") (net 26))
 (segment (start 127.01 65.89) (end 137.81 65.89) (width 1.27) (layer "B.Cu") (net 26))
 (segment (start 141.32 62.38) (end 152.64 62.38) (width 1.27) (layer "B.Cu") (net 26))
 (segment (start 137.69 57.83) (end 142.23 57.83) (width 1.27) (layer "F.Cu") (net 22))
 (via (at 137.69 57.83) (size 2) (drill 0.7) (layers "F.Cu" "B.Cu") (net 22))
 (via (at 142.23 57.83) (size 2) (drill 0.7) (layers "F.Cu" "B.Cu") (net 22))
 (segment (start 137.69 62.43) (end 136.4 63.72) (width 1.27) (layer "B.Cu") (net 22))
 (segment (start 137.69 57.83) (end 137.69 62.43) (width 1.27) (layer "B.Cu") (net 22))
 (segment (start 126.46 56.77) (end 127.59 55.64) (width 1.27) (layer "B.Cu") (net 22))
 (segment (start 147.83 57.83) (end 142.23 57.83) (width 1.27) (layer "B.Cu") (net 22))
 (segment (start 152.64 54.76) (end 150.9 54.76) (width 1.27) (layer "B.Cu") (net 22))
 (segment (start 128.03 63.72) (end 126.46 62.15) (width 1.27) (layer "B.Cu") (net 22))
 (segment (start 136.4 63.72) (end 128.03 63.72) (width 1.27) (layer "B.Cu") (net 22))
 (segment (start 127.59 55.64) (end 132.247 55.64) (width 1.27) (layer "B.Cu") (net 22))
 (segment (start 126.46 62.15) (end 126.46 56.77) (width 1.27) (layer "B.Cu") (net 22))
 (segment (start 148.25 57.41) (end 147.83 57.83) (width 1.27) (layer "B.Cu") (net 22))
 (segment (start 150.9 54.76) (end 148.25 57.41) (width 1.27) (layer "B.Cu") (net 22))
 (segment (start 175.97 85.24) (end 170.42 85.24) (width 1.27) (layer "B.Cu") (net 27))
 (segment (start 138.72 55.63) (end 139.7 56.61) (width 1.27) (layer "B.Cu") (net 21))
 (segment (start 139.7 56.61) (end 139.7 58.94) (width 1.27) (layer "B.Cu") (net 21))
 (segment (start 139.7 58.94) (end 140.61 59.85) (width 1.27) (layer "B.Cu") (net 21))
 (segment (start 140.61 59.85) (end 140.62 59.84) (width 1.27) (layer "B.Cu") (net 21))
 (segment (start 134.81 55.63) (end 138.72 55.63) (width 1.27) (layer "B.Cu") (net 21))
 (segment (start 140.62 59.84) (end 152.64 59.84) (width 1.27) (layer "B.Cu") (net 21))
 (segment (start 128.14 53.1) (end 126.77 51.73) (width 1.27) (layer "B.Cu") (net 24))
 (segment (start 142.95 49.68) (end 152.64 49.68) (width 1.27) (layer "B.Cu") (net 24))
 (segment (start 126.77 51.73) (end 126.77 49.13) (width 1.27) (layer "B.Cu") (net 24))
 (segment (start 128.12 47.78) (end 141.05 47.78) (width 1.27) (layer "B.Cu") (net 24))
 (segment (start 141.05 47.78) (end 142.95 49.68) (width 1.27) (layer "B.Cu") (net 24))
 (segment (start 126.77 49.13) (end 128.12 47.78) (width 1.27) (layer "B.Cu") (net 24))
 (segment (start 132.247 53.1) (end 128.14 53.1) (width 1.27) (layer "B.Cu") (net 24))
 (segment (start 139.09 67.9) (end 142.07 64.92) (width 1.27) (layer "B.Cu") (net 6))
 (segment (start 142.07 64.92) (end 144.7 64.92) (width 1.27) (layer "B.Cu") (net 6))
 (segment (start 134.74 74.6) (end 136.75 74.6) (width 1.27) (layer "B.Cu") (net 6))
 (segment (start 139.09 72.26) (end 139.09 67.9) (width 1.27) (layer "B.Cu") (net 6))
 (segment (start 136.75 74.6) (end 139.09 72.26) (width 1.27) (layer "B.Cu") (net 6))
 (segment (start 144.7 64.92) (end 152.64 64.92) (width 1.27) (layer "B.Cu") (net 6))
 (segment (start 139.41 50.55) (end 134.81 50.55) (width 1.27) (layer "B.Cu") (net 25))
 (segment (start 152.64 52.22) (end 141.08 52.22) (width 1.27) (layer "B.Cu") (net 25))
 (segment (start 141.08 52.22) (end 139.41 50.55) (width 1.27) (layer "B.Cu") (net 25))
 (segment (start 144.67 54.96) (end 144.67 47.14) (width 1.27) (layer "F.Cu") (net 23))
 (via (at 144.67 47.14) (size 2) (drill 0.7) (layers "F.Cu" "B.Cu") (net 23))
 (via (at 144.67 54.96) (size 2) (drill 0.7) (layers "F.Cu" "B.Cu") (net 23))
 (segment (start 141.1 54.96) (end 139.24 53.1) (width 1.27) (layer "B.Cu") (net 23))
 (segment (start 144.67 54.96) (end 141.1 54.96) (width 1.27) (layer "B.Cu") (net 23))
 (segment (start 139.24 53.1) (end 134.787 53.1) (width 1.27) (layer "B.Cu") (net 23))
 (segment (start 152.64 47.14) (end 144.67 47.14) (width 1.27) (layer "B.Cu") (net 23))
 (segment (start 152.63 42.07) (end 152.64 42.06) (width 1.27) (layer "B.Cu") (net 18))
 (segment (start 144.71 42.07) (end 152.63 42.07) (width 1.27) (layer "B.Cu") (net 18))
 (segment (start 170.44 75.1) (end 170.42 75.08) (width 1.27) (layer "B.Cu") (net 10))
 (segment (start 179.06 75.1) (end 170.44 75.1) (width 1.27) (layer "B.Cu") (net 10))
 (segment (start 170.44 77.64) (end 170.42 77.62) (width 1.27) (layer "B.Cu") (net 12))
 (segment (start 179.06 77.64) (end 170.44 77.64) (width 1.27) (layer "B.Cu") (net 12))
 (segment (start 179.01 80.17) (end 184.89 80.17) (width 1.27) (layer "F.Cu") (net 11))
 (segment (start 184.89 80.17) (end 184.94 80.12) (width 1.27) (layer "F.Cu") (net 11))
 (via (at 179.01 80.17) (size 2) (drill 0.7) (layers "F.Cu" "B.Cu") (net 11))
 (via (at 184.94 80.12) (size 2) (drill 0.7) (layers "F.Cu" "B.Cu") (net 11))
 (segment (start 170.43 80.17) (end 170.42 80.16) (width 1.27) (layer "B.Cu") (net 11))
 (segment (start 184.94 80.12) (end 184.94 76.52) (width 1.27) (layer "B.Cu") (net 11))
 (segment (start 183.52 75.1) (end 181.6 75.1) (width 1.27) (layer "B.Cu") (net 11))
 (segment (start 184.94 76.52) (end 183.52 75.1) (width 1.27) (layer "B.Cu") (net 11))
 (segment (start 179.01 80.17) (end 170.43 80.17) (width 1.27) (layer "B.Cu") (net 11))
 (segment (start 185.905 64.885) (end 170.455 64.885) (width 1.27) (layer "B.Cu") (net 16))
 (segment (start 170.455 64.885) (end 170.42 64.92) (width 1.27) (layer "B.Cu") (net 16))
 (segment (start 144.71 39.53) (end 152.63 39.53) (width 1.27) (layer "B.Cu") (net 17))
 (segment (start 152.63 39.53) (end 152.64 39.52) (width 1.27) (layer "B.Cu") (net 17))
 (segment (start 196.01 67.15) (end 200.18 67.15) (width 1.27) (layer "B.Cu") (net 8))
 (segment (start 200.18 67.15) (end 200.42 67.39) (width 1.27) (layer "B.Cu") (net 8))
 (segment (start 145.15 86.22) (end 145.15 84.64) (width 1.27) (layer "B.Cu") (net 13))
 (segment (start 141.6 81.09) (end 138.22 81.09) (width 1.27) (layer "B.Cu") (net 13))
 (segment (start 145.15 84.64) (end 141.6 81.09) (width 1.27) (layer "B.Cu") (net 13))
 (segment (start 200.42 74.62) (end 198.28 72.48) (width 1.27) (layer "B.Cu") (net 15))
 (segment (start 198.28 72.48) (end 194.28 72.48) (width 1.27) (layer "B.Cu") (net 15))
 (segment (start 200.42 77.55) (end 200.42 74.62) (width 1.27) (layer "B.Cu") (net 15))
 (segment (start 186.13 85.24) (end 186.13 83.13) (width 1.27) (layer "B.Cu") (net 19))
 (segment (start 186.13 83.13) (end 190 79.26) (width 1.27) (layer "B.Cu") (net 19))
 (segment (start 190 75.02) (end 194.28 75.02) (width 1.27) (layer "B.Cu") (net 19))
 (segment (start 190 79.26) (end 190 75.02) (width 1.27) (layer "B.Cu") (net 19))
 (segment (start 128.82 58.25) (end 128.83 58.26) (width 1.27) (layer "F.Cu") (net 20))
 (segment (start 121.88 58.25) (end 128.82 58.25) (width 1.27) (layer "F.Cu") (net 20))
 (segment (start 121.81 58.18) (end 121.88 58.25) (width 1.27) (layer "F.Cu") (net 20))
 (via (at 121.81 58.18) (size 2) (drill 0.7) (layers "F.Cu" "B.Cu") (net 20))
 (via (at 128.83 58.26) (size 2) (drill 0.7) (layers "F.Cu" "B.Cu") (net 20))
 (segment (start 132.247 58.18) (end 128.91 58.18) (width 1.27) (layer "B.Cu") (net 20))
 (segment (start 128.91 58.18) (end 128.83 58.26) (width 1.27) (layer "B.Cu") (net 20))
 (segment (start 121.81 58.18) (end 121.8 58.19) (width 1.27) (layer "B.Cu") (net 20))
 (segment (start 121.8 58.19) (end 119.35 58.19) (width 1.27) (layer "B.Cu") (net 20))
 (segment (start 185.905 62.345) (end 185.905 54.875) (width 1.27) (layer "B.Cu") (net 5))
 (segment (start 185.905 54.875) (end 185.99 54.79) (width 1.27) (layer "B.Cu") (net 5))
 (segment (start 191.0547 44.63) (end 192.4812 43.2035) (width 1.27) (layer "B.Cu") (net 3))
 (segment (start 185.99 44.63) (end 191.0547 44.63) (width 1.27) (layer "B.Cu") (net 3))
 (segment (start 193.1742 52.25) (end 193.1793 52.2551) (width 1.27) (layer "B.Cu") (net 4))
 (segment (start 185.99 52.25) (end 193.1742 52.25) (width 1.27) (layer "B.Cu") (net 4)))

